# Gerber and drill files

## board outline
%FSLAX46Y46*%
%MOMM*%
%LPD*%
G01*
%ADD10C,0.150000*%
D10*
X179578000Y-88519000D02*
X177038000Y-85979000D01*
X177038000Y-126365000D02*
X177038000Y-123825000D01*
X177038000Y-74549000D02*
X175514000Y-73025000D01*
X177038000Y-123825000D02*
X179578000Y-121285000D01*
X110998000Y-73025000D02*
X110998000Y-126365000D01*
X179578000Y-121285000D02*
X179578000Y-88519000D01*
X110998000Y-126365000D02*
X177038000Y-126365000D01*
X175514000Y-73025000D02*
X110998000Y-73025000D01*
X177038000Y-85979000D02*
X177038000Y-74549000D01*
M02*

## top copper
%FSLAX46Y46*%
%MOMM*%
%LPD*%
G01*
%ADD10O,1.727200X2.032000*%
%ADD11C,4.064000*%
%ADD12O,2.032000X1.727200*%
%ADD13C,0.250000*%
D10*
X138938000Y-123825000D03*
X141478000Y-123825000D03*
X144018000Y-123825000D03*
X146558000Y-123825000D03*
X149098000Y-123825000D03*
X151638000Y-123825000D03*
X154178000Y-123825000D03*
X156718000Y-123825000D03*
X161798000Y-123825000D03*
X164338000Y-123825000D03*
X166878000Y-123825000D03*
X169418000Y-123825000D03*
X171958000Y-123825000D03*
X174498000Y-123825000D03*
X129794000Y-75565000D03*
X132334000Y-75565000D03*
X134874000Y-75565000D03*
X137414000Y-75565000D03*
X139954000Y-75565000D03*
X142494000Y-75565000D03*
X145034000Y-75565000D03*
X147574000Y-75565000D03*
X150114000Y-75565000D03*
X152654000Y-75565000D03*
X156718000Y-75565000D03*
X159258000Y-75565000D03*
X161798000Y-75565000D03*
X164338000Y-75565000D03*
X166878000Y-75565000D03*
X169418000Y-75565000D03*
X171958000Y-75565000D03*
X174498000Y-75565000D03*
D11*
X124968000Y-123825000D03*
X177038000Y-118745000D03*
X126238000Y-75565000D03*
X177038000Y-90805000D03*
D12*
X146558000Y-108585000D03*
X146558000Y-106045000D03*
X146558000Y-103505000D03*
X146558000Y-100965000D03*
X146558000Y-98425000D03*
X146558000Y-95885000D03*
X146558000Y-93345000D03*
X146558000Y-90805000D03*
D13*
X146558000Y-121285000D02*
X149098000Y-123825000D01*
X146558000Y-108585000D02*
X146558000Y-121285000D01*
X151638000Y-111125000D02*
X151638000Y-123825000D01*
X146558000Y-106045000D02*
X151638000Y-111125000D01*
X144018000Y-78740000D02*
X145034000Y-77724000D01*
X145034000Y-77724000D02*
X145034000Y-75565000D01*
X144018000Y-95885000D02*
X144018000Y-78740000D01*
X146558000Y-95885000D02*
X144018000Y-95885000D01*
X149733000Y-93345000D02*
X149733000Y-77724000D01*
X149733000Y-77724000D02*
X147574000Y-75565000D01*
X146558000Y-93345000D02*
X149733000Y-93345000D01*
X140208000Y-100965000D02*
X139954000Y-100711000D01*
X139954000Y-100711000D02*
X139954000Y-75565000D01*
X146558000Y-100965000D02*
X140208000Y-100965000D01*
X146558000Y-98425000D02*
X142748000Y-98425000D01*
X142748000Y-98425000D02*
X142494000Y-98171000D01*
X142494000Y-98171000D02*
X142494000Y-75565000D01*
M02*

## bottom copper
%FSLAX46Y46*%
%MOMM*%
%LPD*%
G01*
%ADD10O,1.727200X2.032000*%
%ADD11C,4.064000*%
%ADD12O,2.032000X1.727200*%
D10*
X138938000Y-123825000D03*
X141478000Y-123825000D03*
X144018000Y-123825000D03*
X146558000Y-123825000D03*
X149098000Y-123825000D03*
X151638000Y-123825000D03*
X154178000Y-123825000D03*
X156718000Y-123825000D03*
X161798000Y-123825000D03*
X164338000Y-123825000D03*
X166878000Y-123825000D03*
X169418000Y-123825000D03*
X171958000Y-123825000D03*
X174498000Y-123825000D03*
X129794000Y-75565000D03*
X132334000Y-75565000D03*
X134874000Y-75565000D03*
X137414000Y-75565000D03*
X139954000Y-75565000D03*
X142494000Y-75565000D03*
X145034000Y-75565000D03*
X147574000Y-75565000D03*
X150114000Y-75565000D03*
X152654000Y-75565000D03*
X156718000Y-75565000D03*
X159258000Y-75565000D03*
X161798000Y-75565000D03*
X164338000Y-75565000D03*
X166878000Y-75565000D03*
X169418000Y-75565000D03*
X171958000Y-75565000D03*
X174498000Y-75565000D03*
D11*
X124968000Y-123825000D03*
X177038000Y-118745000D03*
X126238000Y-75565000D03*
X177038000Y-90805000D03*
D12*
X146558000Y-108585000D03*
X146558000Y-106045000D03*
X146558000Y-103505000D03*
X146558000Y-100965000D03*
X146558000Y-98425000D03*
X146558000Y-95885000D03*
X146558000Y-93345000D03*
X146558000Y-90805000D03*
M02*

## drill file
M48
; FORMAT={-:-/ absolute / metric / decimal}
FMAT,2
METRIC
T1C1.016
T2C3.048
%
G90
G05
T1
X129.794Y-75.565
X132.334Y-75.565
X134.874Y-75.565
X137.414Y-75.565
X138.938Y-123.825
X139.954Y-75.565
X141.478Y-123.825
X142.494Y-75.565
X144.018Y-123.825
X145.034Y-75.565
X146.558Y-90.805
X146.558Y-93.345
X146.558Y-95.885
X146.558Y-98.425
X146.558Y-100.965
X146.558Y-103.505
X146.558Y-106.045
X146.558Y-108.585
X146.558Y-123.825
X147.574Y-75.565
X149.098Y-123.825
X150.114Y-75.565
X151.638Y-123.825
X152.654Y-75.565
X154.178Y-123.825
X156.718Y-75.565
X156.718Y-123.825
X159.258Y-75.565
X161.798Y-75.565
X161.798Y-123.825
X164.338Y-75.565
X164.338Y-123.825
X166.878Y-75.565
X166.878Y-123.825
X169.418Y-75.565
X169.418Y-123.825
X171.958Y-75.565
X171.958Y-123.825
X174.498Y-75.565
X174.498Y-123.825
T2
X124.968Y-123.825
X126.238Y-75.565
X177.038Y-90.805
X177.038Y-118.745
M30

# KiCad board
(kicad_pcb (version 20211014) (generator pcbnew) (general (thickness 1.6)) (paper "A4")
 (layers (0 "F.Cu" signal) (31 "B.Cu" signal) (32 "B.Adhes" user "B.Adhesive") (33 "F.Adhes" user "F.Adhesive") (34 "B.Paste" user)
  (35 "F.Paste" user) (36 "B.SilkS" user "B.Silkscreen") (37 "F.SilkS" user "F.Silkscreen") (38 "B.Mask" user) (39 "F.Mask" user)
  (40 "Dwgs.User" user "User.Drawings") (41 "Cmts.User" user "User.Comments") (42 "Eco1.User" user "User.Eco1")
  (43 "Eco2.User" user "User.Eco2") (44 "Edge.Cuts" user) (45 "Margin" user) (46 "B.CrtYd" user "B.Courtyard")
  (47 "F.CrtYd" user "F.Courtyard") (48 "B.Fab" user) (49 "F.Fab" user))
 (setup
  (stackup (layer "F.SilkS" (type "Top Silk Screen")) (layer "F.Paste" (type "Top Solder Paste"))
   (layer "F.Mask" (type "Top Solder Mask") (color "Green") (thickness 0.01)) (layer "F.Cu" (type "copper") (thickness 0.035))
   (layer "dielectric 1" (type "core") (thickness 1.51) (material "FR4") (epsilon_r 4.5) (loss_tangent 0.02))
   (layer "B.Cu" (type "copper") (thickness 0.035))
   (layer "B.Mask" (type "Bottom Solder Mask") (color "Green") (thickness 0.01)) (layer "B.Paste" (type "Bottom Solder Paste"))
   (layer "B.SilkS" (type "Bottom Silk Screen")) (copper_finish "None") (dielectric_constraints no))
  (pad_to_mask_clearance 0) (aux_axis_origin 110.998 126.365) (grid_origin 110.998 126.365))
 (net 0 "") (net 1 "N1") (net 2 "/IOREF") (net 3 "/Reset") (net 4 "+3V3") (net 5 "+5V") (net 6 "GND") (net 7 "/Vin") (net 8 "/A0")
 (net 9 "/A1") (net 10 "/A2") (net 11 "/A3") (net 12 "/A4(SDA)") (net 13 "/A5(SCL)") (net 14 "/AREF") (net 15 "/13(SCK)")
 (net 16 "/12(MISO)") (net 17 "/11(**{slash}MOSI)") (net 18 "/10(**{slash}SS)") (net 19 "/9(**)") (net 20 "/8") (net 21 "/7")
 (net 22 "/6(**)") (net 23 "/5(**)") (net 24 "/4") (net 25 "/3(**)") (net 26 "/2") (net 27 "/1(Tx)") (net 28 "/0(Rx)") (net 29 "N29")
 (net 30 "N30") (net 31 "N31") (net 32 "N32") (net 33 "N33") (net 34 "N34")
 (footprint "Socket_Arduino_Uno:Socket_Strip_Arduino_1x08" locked (layer "F.Cu") (at 138.938 123.825)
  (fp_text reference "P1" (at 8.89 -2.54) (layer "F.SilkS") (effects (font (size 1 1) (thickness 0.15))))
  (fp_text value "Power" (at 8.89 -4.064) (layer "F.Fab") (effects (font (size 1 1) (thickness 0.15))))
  (pad "1" thru_hole oval locked (at 0 0) (size 1.7272 2.032) (drill 1.016) (layers *.Cu *.Mask "F.SilkS") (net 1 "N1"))
  (pad "2" thru_hole oval locked (at 2.54 0) (size 1.7272 2.032) (drill 1.016) (layers *.Cu *.Mask "F.SilkS") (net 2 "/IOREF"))
  (pad "3" thru_hole oval locked (at 5.08 0) (size 1.7272 2.032) (drill 1.016) (layers *.Cu *.Mask "F.SilkS") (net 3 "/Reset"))
  (pad "4" thru_hole oval locked (at 7.62 0) (size 1.7272 2.032) (drill 1.016) (layers *.Cu *.Mask "F.SilkS") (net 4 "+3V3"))
  (pad "5" thru_hole oval locked (at 10.16 0) (size 1.7272 2.032) (drill 1.016) (layers *.Cu *.Mask "F.SilkS") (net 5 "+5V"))
  (pad "6" thru_hole oval locked (at 12.7 0) (size 1.7272 2.032) (drill 1.016) (layers *.Cu *.Mask "F.SilkS") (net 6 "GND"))
  (pad "7" thru_hole oval locked (at 15.24 0) (size 1.7272 2.032) (drill 1.016) (layers *.Cu *.Mask "F.SilkS") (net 6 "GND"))
  (pad "8" thru_hole oval locked (at 17.78 0) (size 1.7272 2.032) (drill 1.016) (layers *.Cu *.Mask "F.SilkS") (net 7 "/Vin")))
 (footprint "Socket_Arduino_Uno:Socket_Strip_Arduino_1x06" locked (layer "F.Cu") (at 161.798 123.825)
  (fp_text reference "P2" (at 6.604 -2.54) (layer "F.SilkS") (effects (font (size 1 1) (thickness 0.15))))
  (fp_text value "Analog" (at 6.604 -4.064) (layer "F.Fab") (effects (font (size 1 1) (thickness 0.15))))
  (pad "1" thru_hole oval locked (at 0 0) (size 1.7272 2.032) (drill 1.016) (layers *.Cu *.Mask "F.SilkS") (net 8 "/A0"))
  (pad "2" thru_hole oval locked (at 2.54 0) (size 1.7272 2.032) (drill 1.016) (layers *.Cu *.Mask "F.SilkS") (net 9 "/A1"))
  (pad "3" thru_hole oval locked (at 5.08 0) (size 1.7272 2.032) (drill 1.016) (layers *.Cu *.Mask "F.SilkS") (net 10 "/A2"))
  (pad "4" thru_hole oval locked (at 7.62 0) (size 1.7272 2.032) (drill 1.016) (layers *.Cu *.Mask "F.SilkS") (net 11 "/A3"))
  (pad "5" thru_hole oval locked (at 10.16 0) (size 1.7272 2.032) (drill 1.016) (layers *.Cu *.Mask "F.SilkS") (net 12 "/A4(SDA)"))
  (pad "6" thru_hole oval locked (at 12.7 0) (size 1.7272 2.032) (drill 1.016) (layers *.Cu *.Mask "F.SilkS") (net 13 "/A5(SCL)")))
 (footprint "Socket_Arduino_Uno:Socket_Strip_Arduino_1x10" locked (layer "F.Cu") (at 129.794 75.565)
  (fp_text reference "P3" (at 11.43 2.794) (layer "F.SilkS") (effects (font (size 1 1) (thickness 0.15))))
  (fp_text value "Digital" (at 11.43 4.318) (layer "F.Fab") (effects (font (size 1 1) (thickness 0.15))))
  (pad "1" thru_hole oval locked (at 0 0) (size 1.7272 2.032) (drill 1.016) (layers *.Cu *.Mask "F.SilkS") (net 13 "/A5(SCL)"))
  (pad "2" thru_hole oval locked (at 2.54 0) (size 1.7272 2.032) (drill 1.016) (layers *.Cu *.Mask "F.SilkS") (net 12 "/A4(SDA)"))
  (pad "3" thru_hole oval locked (at 5.08 0) (size 1.7272 2.032) (drill 1.016) (layers *.Cu *.Mask "F.SilkS") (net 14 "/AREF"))
  (pad "4" thru_hole oval locked (at 7.62 0) (size 1.7272 2.032) (drill 1.016) (layers *.Cu *.Mask "F.SilkS") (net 6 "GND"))
  (pad "5" thru_hole oval locked (at 10.16 0) (size 1.7272 2.032) (drill 1.016) (layers *.Cu *.Mask "F.SilkS") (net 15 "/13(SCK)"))
  (pad "6" thru_hole oval locked (at 12.7 0) (size 1.7272 2.032) (drill 1.016) (layers *.Cu *.Mask "F.SilkS") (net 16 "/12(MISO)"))
  (pad "7" thru_hole oval locked (at 15.24 0) (size 1.7272 2.032) (drill 1.016) (layers *.Cu *.Mask "F.SilkS") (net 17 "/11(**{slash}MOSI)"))
  (pad "8" thru_hole oval locked (at 17.78 0) (size 1.7272 2.032) (drill 1.016) (layers *.Cu *.Mask "F.SilkS") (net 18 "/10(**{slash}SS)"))
  (pad "9" thru_hole oval locked (at 20.32 0) (size 1.7272 2.032) (drill 1.016) (layers *.Cu *.Mask "F.SilkS") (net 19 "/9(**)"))
  (pad "10" thru_hole oval locked (at 22.86 0) (size 1.7272 2.032) (drill 1.016) (layers *.Cu *.Mask "F.SilkS") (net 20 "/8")))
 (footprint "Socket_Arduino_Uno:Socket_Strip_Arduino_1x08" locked (layer "F.Cu") (at 156.718 75.565)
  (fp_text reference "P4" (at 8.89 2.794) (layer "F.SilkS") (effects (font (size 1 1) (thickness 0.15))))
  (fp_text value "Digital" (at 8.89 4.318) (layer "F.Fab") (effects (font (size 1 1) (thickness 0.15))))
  (pad "1" thru_hole oval locked (at 0 0) (size 1.7272 2.032) (drill 1.016) (layers *.Cu *.Mask "F.SilkS") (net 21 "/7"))
  (pad "2" thru_hole oval locked (at 2.54 0) (size 1.7272 2.032) (drill 1.016) (layers *.Cu *.Mask "F.SilkS") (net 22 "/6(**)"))
  (pad "3" thru_hole oval locked (at 5.08 0) (size 1.7272 2.032) (drill 1.016) (layers *.Cu *.Mask "F.SilkS") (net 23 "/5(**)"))
  (pad "4" thru_hole oval locked (at 7.62 0) (size 1.7272 2.032) (drill 1.016) (layers *.Cu *.Mask "F.SilkS") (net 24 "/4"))
  (pad "5" thru_hole oval locked (at 10.16 0) (size 1.7272 2.032) (drill 1.016) (layers *.Cu *.Mask "F.SilkS") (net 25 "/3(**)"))
  (pad "6" thru_hole oval locked (at 12.7 0) (size 1.7272 2.032) (drill 1.016) (layers *.Cu *.Mask "F.SilkS") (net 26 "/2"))
  (pad "7" thru_hole oval locked (at 15.24 0) (size 1.7272 2.032) (drill 1.016) (layers *.Cu *.Mask "F.SilkS") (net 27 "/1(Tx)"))
  (pad "8" thru_hole oval locked (at 17.78 0) (size 1.7272 2.032) (drill 1.016) (layers *.Cu *.Mask "F.SilkS") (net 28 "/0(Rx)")))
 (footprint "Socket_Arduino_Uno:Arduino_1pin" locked (layer "F.Cu") (at 124.968 123.825)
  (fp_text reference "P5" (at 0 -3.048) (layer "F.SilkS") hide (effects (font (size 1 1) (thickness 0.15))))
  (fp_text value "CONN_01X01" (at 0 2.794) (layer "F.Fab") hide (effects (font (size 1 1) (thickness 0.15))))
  (pad "1" thru_hole circle locked (at 0 0) (size 4.064 4.064) (drill 3.048) (layers *.Cu *.Mask "F.SilkS") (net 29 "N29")))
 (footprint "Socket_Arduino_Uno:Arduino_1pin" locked (layer "F.Cu") (at 177.038 118.745)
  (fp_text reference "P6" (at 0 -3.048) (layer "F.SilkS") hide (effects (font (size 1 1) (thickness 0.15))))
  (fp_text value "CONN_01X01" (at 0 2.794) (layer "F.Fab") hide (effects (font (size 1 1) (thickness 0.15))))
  (pad "1" thru_hole circle locked (at 0 0) (size 4.064 4.064) (drill 3.048) (layers *.Cu *.Mask "F.SilkS") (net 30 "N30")))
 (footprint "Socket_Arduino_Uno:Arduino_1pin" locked (layer "F.Cu") (at 126.238 75.565)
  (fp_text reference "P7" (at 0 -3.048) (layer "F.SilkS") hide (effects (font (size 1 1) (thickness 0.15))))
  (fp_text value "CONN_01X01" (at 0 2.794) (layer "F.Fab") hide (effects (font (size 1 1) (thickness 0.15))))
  (pad "1" thru_hole circle locked (at 0 0) (size 4.064 4.064) (drill 3.048) (layers *.Cu *.Mask "F.SilkS") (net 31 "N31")))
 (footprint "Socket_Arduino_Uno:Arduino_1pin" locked (layer "F.Cu") (at 177.038 90.805)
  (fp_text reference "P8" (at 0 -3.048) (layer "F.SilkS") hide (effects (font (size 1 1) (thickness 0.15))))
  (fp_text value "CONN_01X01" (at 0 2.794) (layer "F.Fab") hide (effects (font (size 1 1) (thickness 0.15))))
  (pad "1" thru_hole circle locked (at 0 0) (size 4.064 4.064) (drill 3.048) (layers *.Cu *.Mask "F.SilkS") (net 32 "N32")))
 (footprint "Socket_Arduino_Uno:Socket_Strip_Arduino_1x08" (layer "F.Cu") (at 146.558 108.585 90)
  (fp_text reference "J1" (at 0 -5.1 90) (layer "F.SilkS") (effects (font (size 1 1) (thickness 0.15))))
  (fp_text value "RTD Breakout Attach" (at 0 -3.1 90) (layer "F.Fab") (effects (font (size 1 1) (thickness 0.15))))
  (pad "1" thru_hole oval locked (at 0 0 90) (size 1.7272 2.032) (drill 1.016) (layers *.Cu *.Mask "F.SilkS") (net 5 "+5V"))
  (pad "2" thru_hole oval locked (at 2.54 0 90) (size 1.7272 2.032) (drill 1.016) (layers *.Cu *.Mask "F.SilkS") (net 6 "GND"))
  (pad "3" thru_hole oval locked (at 5.08 0 90) (size 1.7272 2.032) (drill 1.016) (layers *.Cu *.Mask "F.SilkS") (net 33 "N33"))
  (pad "4" thru_hole oval locked (at 7.62 0 90) (size 1.7272 2.032) (drill 1.016) (layers *.Cu *.Mask "F.SilkS") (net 15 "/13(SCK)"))
  (pad "5" thru_hole oval locked (at 10.16 0 90) (size 1.7272 2.032) (drill 1.016) (layers *.Cu *.Mask "F.SilkS") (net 16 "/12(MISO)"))
  (pad "6" thru_hole oval locked (at 12.7 0 90) (size 1.7272 2.032) (drill 1.016) (layers *.Cu *.Mask "F.SilkS")
   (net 17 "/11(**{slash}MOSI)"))
  (pad "7" thru_hole oval locked (at 15.24 0 90) (size 1.7272 2.032) (drill 1.016) (layers *.Cu *.Mask "F.SilkS")
   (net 18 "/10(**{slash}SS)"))
  (pad "8" thru_hole oval locked (at 17.78 0 90) (size 1.7272 2.032) (drill 1.016) (layers *.Cu *.Mask "F.SilkS") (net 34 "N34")))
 (gr_line (start 179.578 88.519) (end 177.038 85.979) (layer "Edge.Cuts") (width 0.15))
 (gr_line (start 177.038 126.365) (end 177.038 123.825) (layer "Edge.Cuts") (width 0.15))
 (gr_line (start 177.038 74.549) (end 175.514 73.025) (layer "Edge.Cuts") (width 0.15))
 (gr_line (start 177.038 123.825) (end 179.578 121.285) (layer "Edge.Cuts") (width 0.15))
 (gr_line (start 110.998 73.025) (end 110.998 126.365) (layer "Edge.Cuts") (width 0.15))
 (gr_line (start 179.578 121.285) (end 179.578 88.519) (layer "Edge.Cuts") (width 0.15))
 (gr_line (start 110.998 126.365) (end 177.038 126.365) (layer "Edge.Cuts") (width 0.15))
 (gr_line (start 175.514 73.025) (end 110.998 73.025) (layer "Edge.Cuts") (width 0.15))
 (gr_line (start 177.038 85.979) (end 177.038 74.549) (layer "Edge.Cuts") (width 0.15))
 (segment (start 146.558 121.285) (end 149.098 123.825) (width 0.25) (layer "F.Cu") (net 5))
 (segment (start 146.558 108.585) (end 146.558 121.285) (width 0.25) (layer "F.Cu") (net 5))
 (segment (start 151.638 111.125) (end 151.638 123.825) (width 0.25) (layer "F.Cu") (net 6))
 (segment (start 146.558 106.045) (end 151.638 111.125) (width 0.25) (layer "F.Cu") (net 6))
 (segment (start 144.018 78.74) (end 145.034 77.724) (width 0.25) (layer "F.Cu") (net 17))
 (segment (start 145.034 77.724) (end 145.034 75.565) (width 0.25) (layer "F.Cu") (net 17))
 (segment (start 144.018 95.885) (end 144.018 78.74) (width 0.25) (layer "F.Cu") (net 17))
 (segment (start 146.558 95.885) (end 144.018 95.885) (width 0.25) (layer "F.Cu") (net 17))
 (segment (start 149.733 93.345) (end 149.733 77.724) (width 0.25) (layer "F.Cu") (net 18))
 (segment (start 149.733 77.724) (end 147.574 75.565) (width 0.25) (layer "F.Cu") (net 18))
 (segment (start 146.558 93.345) (end 149.733 93.345) (width 0.25) (layer "F.Cu") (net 18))
 (segment (start 140.208 100.965) (end 139.954 100.711) (width 0.25) (layer "F.Cu") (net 15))
 (segment (start 139.954 100.711) (end 139.954 75.565) (width 0.25) (layer "F.Cu") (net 15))
 (segment (start 146.558 100.965) (end 140.208 100.965) (width 0.25) (layer "F.Cu") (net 15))
 (segment (start 146.558 98.425) (end 142.748 98.425) (width 0.25) (layer "F.Cu") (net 16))
 (segment (start 142.748 98.425) (end 142.494 98.171) (width 0.25) (layer "F.Cu") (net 16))
 (segment (start 142.494 98.171) (end 142.494 75.565) (width 0.25) (layer "F.Cu") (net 16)))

